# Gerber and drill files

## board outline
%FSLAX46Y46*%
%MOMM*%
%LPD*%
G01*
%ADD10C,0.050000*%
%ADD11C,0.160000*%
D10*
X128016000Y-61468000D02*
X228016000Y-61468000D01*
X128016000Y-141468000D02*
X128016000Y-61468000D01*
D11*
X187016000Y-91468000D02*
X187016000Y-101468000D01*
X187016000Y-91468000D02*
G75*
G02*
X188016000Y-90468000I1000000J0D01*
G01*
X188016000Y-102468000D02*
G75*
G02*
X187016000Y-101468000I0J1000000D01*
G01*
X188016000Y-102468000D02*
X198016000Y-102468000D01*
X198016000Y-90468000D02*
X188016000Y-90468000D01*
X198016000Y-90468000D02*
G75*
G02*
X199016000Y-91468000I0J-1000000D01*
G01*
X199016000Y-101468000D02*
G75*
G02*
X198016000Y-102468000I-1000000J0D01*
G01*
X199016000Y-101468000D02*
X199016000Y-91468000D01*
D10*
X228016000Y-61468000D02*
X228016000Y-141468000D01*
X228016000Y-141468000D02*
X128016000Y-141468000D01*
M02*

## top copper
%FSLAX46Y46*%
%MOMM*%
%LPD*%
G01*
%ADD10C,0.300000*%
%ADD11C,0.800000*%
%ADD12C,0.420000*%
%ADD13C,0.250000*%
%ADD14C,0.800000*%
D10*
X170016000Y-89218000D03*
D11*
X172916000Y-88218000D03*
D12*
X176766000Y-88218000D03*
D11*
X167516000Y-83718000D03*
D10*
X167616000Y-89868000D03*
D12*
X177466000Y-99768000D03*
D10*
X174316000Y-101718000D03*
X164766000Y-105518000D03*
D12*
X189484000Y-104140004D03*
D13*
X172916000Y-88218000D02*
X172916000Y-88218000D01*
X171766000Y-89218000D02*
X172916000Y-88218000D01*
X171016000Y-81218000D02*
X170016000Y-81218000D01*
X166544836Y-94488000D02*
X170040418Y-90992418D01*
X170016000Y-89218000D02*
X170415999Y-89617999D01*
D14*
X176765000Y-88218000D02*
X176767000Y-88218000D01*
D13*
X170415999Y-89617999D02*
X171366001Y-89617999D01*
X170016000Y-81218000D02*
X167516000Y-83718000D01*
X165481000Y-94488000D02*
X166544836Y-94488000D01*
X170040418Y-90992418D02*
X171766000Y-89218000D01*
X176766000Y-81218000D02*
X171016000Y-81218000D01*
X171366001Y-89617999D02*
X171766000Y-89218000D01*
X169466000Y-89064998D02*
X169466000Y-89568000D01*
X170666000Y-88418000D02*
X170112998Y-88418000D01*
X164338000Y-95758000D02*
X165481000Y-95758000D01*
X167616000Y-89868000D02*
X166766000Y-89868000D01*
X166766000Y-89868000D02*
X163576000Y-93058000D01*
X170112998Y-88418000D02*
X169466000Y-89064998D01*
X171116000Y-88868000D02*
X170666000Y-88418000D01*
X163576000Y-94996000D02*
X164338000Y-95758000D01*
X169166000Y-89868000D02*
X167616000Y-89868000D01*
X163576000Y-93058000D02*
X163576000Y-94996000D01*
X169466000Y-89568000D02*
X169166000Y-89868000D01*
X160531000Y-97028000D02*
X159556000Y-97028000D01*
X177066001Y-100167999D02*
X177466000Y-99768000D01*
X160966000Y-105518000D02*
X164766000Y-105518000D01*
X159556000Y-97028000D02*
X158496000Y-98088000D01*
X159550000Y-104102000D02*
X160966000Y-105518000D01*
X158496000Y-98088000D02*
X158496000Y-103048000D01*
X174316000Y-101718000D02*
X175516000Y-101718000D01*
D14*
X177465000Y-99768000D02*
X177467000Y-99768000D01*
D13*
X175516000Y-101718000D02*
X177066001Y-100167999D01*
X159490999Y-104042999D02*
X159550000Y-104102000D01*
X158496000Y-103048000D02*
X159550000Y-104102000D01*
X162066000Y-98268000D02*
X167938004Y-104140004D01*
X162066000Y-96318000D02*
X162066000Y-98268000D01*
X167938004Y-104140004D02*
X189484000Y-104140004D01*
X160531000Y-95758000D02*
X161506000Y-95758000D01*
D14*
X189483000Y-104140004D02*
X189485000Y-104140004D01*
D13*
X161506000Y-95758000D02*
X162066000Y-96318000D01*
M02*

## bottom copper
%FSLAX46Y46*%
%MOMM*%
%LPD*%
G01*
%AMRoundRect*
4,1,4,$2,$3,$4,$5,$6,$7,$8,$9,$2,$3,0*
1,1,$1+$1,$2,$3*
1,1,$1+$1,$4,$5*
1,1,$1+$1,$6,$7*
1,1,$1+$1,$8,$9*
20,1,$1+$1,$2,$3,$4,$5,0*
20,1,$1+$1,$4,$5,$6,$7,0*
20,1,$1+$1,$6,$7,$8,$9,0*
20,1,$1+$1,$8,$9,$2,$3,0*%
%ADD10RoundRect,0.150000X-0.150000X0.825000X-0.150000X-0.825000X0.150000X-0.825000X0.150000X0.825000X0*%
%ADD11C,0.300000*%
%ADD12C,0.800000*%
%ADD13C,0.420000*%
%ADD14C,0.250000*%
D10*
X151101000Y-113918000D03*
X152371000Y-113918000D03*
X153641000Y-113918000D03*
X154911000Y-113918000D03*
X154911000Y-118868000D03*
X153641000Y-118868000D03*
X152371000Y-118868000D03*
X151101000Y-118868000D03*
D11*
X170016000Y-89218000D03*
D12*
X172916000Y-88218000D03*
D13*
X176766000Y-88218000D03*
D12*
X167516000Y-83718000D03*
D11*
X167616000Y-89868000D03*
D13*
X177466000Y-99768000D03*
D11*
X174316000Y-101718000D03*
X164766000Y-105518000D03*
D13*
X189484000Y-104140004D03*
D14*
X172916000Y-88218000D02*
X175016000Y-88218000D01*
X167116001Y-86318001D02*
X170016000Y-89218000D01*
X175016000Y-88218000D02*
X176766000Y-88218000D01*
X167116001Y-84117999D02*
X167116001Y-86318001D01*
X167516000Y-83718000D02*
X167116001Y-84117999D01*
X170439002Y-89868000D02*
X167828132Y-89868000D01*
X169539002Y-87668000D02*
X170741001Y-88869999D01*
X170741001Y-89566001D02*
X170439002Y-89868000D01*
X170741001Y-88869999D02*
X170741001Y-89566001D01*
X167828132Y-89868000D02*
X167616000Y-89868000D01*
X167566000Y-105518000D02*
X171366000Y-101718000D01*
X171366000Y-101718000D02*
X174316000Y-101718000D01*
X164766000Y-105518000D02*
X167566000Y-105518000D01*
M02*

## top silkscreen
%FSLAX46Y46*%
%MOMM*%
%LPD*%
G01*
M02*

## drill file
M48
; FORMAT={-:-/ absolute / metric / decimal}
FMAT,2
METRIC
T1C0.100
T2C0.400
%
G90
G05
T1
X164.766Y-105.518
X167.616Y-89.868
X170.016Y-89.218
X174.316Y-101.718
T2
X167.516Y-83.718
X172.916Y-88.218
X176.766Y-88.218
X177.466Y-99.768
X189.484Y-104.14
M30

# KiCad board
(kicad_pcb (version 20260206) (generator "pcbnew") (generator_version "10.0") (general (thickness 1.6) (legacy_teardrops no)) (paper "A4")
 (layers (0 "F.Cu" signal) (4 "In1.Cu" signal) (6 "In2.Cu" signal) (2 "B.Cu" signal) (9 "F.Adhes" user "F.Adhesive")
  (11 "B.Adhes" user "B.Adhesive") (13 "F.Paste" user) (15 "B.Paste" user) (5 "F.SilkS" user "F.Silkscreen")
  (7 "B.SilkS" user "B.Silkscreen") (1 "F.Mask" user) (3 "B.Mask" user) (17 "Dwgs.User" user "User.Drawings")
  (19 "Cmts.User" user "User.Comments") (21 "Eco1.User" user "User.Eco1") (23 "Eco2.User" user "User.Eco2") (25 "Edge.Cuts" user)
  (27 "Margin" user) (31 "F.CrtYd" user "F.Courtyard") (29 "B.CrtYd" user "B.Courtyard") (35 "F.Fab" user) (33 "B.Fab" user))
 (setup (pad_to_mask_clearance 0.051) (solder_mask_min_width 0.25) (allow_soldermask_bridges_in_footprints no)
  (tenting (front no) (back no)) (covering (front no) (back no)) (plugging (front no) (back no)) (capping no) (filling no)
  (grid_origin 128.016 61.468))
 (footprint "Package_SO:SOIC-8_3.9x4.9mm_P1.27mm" (layer "B.Cu") (at 153.006 116.393 -90)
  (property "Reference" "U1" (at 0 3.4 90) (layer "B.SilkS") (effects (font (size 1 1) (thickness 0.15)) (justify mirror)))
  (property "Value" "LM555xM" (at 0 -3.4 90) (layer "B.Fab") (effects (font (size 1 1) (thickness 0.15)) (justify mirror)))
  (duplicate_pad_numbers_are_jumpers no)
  (pad "1" smd roundrect (at -2.475 1.905 270) (size 1.95 0.6) (layers "B.Cu" "B.Mask" "B.Paste") (roundrect_rratio 0.25)
   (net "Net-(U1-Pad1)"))
  (pad "2" smd roundrect (at -2.475 0.635 270) (size 1.95 0.6) (layers "B.Cu" "B.Mask" "B.Paste") (roundrect_rratio 0.25)
   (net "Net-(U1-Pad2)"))
  (pad "3" smd roundrect (at -2.475 -0.635 270) (size 1.95 0.6) (layers "B.Cu" "B.Mask" "B.Paste") (roundrect_rratio 0.25)
   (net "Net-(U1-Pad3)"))
  (pad "4" smd roundrect (at -2.475 -1.905 270) (size 1.95 0.6) (layers "B.Cu" "B.Mask" "B.Paste") (roundrect_rratio 0.25)
   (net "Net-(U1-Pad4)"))
  (pad "5" smd roundrect (at 2.475 -1.905 270) (size 1.95 0.6) (layers "B.Cu" "B.Mask" "B.Paste") (roundrect_rratio 0.25)
   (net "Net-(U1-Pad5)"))
  (pad "6" smd roundrect (at 2.475 -0.635 270) (size 1.95 0.6) (layers "B.Cu" "B.Mask" "B.Paste") (roundrect_rratio 0.25)
   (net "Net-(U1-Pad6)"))
  (pad "7" smd roundrect (at 2.475 0.635 270) (size 1.95 0.6) (layers "B.Cu" "B.Mask" "B.Paste") (roundrect_rratio 0.25)
   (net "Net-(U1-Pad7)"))
  (pad "8" smd roundrect (at 2.475 1.905 270) (size 1.95 0.6) (layers "B.Cu" "B.Mask" "B.Paste") (roundrect_rratio 0.25)
   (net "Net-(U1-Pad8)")))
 (gr_line (start 128.016 61.468) (end 228.016 61.468) (stroke (width 0.05) (type solid)) (layer "Edge.Cuts"))
 (gr_line (start 128.016 141.468) (end 128.016 61.468) (stroke (width 0.05) (type solid)) (layer "Edge.Cuts"))
 (gr_line (start 187.016 91.468) (end 187.016 101.468) (stroke (width 0.16) (type solid)) (layer "Edge.Cuts"))
 (gr_arc (start 187.016 91.468) (mid 187.308893 90.760893) (end 188.016 90.468) (stroke (width 0.16) (type solid)) (layer "Edge.Cuts"))
 (gr_arc (start 188.016 102.468) (mid 187.308893 102.175107) (end 187.016 101.468) (stroke (width 0.16) (type solid)) (layer "Edge.Cuts"))
 (gr_line (start 188.016 102.468) (end 198.016 102.468) (stroke (width 0.16) (type solid)) (layer "Edge.Cuts"))
 (gr_line (start 198.016 90.468) (end 188.016 90.468) (stroke (width 0.16) (type solid)) (layer "Edge.Cuts"))
 (gr_arc (start 198.016 90.468) (mid 198.723107 90.760893) (end 199.016 91.468) (stroke (width 0.16) (type solid)) (layer "Edge.Cuts"))
 (gr_arc (start 199.016 101.468) (mid 198.723107 102.175107) (end 198.016 102.468) (stroke (width 0.16) (type solid)) (layer "Edge.Cuts"))
 (gr_line (start 199.016 101.468) (end 199.016 91.468) (stroke (width 0.16) (type solid)) (layer "Edge.Cuts"))
 (gr_line (start 228.016 61.468) (end 228.016 141.468) (stroke (width 0.05) (type solid)) (layer "Edge.Cuts"))
 (gr_line (start 228.016 141.468) (end 128.016 141.468) (stroke (width 0.05) (type solid)) (layer "Edge.Cuts"))
 (segment (start 172.916 88.218) (end 172.916 88.218) (width 0.25) (layer "F.Cu") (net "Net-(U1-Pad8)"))
 (segment (start 171.766 89.218) (end 172.916 88.218) (width 0.25) (layer "F.Cu") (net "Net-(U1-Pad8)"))
 (segment (start 171.016 81.218) (end 170.016 81.218) (width 0.25) (layer "F.Cu") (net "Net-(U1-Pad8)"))
 (segment (start 166.544836 94.488) (end 170.040418 90.992418) (width 0.25) (layer "F.Cu") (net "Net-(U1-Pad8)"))
 (segment (start 170.016 89.218) (end 170.415999 89.617999) (width 0.25) (layer "F.Cu") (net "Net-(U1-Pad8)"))
 (segment (start 176.765 88.218) (end 176.767 88.218) (width 0.8) (layer "F.Cu") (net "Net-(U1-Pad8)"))
 (segment (start 170.415999 89.617999) (end 171.366001 89.617999) (width 0.25) (layer "F.Cu") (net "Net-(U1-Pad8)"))
 (segment (start 170.016 81.218) (end 167.516 83.718) (width 0.25) (layer "F.Cu") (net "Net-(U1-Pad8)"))
 (segment (start 165.481 94.488) (end 166.544836 94.488) (width 0.25) (layer "F.Cu") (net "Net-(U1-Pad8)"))
 (segment (start 170.040418 90.992418) (end 171.766 89.218) (width 0.25) (layer "F.Cu") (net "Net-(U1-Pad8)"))
 (segment (start 176.766 81.218) (end 171.016 81.218) (width 0.25) (layer "F.Cu") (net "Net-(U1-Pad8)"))
 (segment (start 171.366001 89.617999) (end 171.766 89.218) (width 0.25) (layer "F.Cu") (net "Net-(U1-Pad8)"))
 (via (at 170.016 89.218) (size 0.3) (drill 0.1) (layers "F.Cu" "B.Cu") (capping no) (covering (front no) (back no))
  (plugging (front no) (back no)) (filling no) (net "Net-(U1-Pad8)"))
 (via (at 172.916 88.218) (size 0.8) (drill 0.4) (layers "F.Cu" "B.Cu") (capping no) (covering (front no) (back no))
  (plugging (front no) (back no)) (filling no) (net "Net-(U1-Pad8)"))
 (via (at 176.766 88.218) (size 0.42) (drill 0.4) (layers "F.Cu" "B.Cu") (capping no) (covering (front no) (back no))
  (plugging (front no) (back no)) (filling no) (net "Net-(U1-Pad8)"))
 (via (at 167.516 83.718) (size 0.8) (drill 0.4) (layers "F.Cu" "B.Cu") (capping no) (covering (front no) (back no))
  (plugging (front no) (back no)) (filling no) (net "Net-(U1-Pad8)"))
 (segment (start 172.916 88.218) (end 175.016 88.218) (width 0.25) (layer "B.Cu") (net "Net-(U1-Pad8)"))
 (segment (start 167.116001 86.318001) (end 170.016 89.218) (width 0.25) (layer "B.Cu") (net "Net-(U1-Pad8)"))
 (segment (start 175.016 88.218) (end 176.766 88.218) (width 0.25) (layer "B.Cu") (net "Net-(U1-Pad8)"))
 (segment (start 167.116001 84.117999) (end 167.116001 86.318001) (width 0.25) (layer "B.Cu") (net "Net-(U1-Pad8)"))
 (segment (start 167.516 83.718) (end 167.116001 84.117999) (width 0.25) (layer "B.Cu") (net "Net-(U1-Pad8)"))
 (segment (start 169.466 89.064998) (end 169.466 89.568) (width 0.25) (layer "F.Cu") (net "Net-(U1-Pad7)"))
 (segment (start 170.666 88.418) (end 170.112998 88.418) (width 0.25) (layer "F.Cu") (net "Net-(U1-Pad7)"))
 (segment (start 164.338 95.758) (end 165.481 95.758) (width 0.25) (layer "F.Cu") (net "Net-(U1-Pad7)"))
 (segment (start 167.616 89.868) (end 166.766 89.868) (width 0.25) (layer "F.Cu") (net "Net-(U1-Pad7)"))
 (segment (start 166.766 89.868) (end 163.576 93.058) (width 0.25) (layer "F.Cu") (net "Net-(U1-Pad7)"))
 (segment (start 170.112998 88.418) (end 169.466 89.064998) (width 0.25) (layer "F.Cu") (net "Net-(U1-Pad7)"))
 (segment (start 171.116 88.868) (end 170.666 88.418) (width 0.25) (layer "F.Cu") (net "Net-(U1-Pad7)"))
 (segment (start 163.576 94.996) (end 164.338 95.758) (width 0.25) (layer "F.Cu") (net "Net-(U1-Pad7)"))
 (segment (start 169.166 89.868) (end 167.616 89.868) (width 0.25) (layer "F.Cu") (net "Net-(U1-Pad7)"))
 (segment (start 163.576 93.058) (end 163.576 94.996) (width 0.25) (layer "F.Cu") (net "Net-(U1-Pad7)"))
 (segment (start 169.466 89.568) (end 169.166 89.868) (width 0.25) (layer "F.Cu") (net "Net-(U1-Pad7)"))
 (via (at 167.616 89.868) (size 0.3) (drill 0.1) (layers "F.Cu" "B.Cu") (capping no) (covering (front no) (back no))
  (plugging (front no) (back no)) (filling no) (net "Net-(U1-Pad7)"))
 (segment (start 170.439002 89.868) (end 167.828132 89.868) (width 0.25) (layer "B.Cu") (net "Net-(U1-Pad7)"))
 (segment (start 169.539002 87.668) (end 170.741001 88.869999) (width 0.25) (layer "B.Cu") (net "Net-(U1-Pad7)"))
 (segment (start 170.741001 89.566001) (end 170.439002 89.868) (width 0.25) (layer "B.Cu") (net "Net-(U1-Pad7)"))
 (segment (start 170.741001 88.869999) (end 170.741001 89.566001) (width 0.25) (layer "B.Cu") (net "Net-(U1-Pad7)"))
 (segment (start 167.828132 89.868) (end 167.616 89.868) (width 0.25) (layer "B.Cu") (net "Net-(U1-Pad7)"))
 (segment (start 160.531 97.028) (end 159.556 97.028) (width 0.25) (layer "F.Cu") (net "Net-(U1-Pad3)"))
 (segment (start 177.066001 100.167999) (end 177.466 99.768) (width 0.25) (layer "F.Cu") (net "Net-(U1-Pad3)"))
 (segment (start 160.966 105.518) (end 164.766 105.518) (width 0.25) (layer "F.Cu") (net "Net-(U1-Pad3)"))
 (segment (start 159.556 97.028) (end 158.496 98.088) (width 0.25) (layer "F.Cu") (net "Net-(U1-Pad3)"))
 (segment (start 159.55 104.102) (end 160.966 105.518) (width 0.25) (layer "F.Cu") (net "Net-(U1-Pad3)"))
 (segment (start 158.496 98.088) (end 158.496 103.048) (width 0.25) (layer "F.Cu") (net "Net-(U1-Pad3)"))
 (segment (start 174.316 101.718) (end 175.516 101.718) (width 0.25) (layer "F.Cu") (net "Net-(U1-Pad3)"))
 (segment (start 177.465 99.768) (end 177.467 99.768) (width 0.8) (layer "F.Cu") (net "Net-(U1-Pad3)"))
 (segment (start 175.516 101.718) (end 177.066001 100.167999) (width 0.25) (layer "F.Cu") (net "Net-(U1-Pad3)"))
 (segment (start 159.490999 104.042999) (end 159.55 104.102) (width 0.25) (layer "F.Cu") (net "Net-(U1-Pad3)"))
 (segment (start 158.496 103.048) (end 159.55 104.102) (width 0.25) (layer "F.Cu") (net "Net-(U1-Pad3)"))
 (via (at 177.466 99.768) (size 0.42) (drill 0.4) (layers "F.Cu" "B.Cu") (capping no) (covering (front no) (back no))
  (plugging (front no) (back no)) (filling no) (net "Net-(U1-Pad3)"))
 (via (at 174.316 101.718) (size 0.3) (drill 0.1) (layers "F.Cu" "B.Cu") (capping no) (covering (front no) (back no))
  (plugging (front no) (back no)) (filling no) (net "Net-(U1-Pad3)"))
 (via (at 164.766 105.518) (size 0.3) (drill 0.1) (layers "F.Cu" "B.Cu") (capping no) (covering (front no) (back no))
  (plugging (front no) (back no)) (filling no) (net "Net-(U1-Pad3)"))
 (segment (start 167.566 105.518) (end 171.366 101.718) (width 0.25) (layer "B.Cu") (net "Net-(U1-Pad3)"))
 (segment (start 171.366 101.718) (end 174.316 101.718) (width 0.25) (layer "B.Cu") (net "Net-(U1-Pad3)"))
 (segment (start 164.766 105.518) (end 167.566 105.518) (width 0.25) (layer "B.Cu") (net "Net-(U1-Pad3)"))
 (segment (start 162.066 98.268) (end 167.938004 104.140004) (width 0.25) (layer "F.Cu") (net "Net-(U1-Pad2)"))
 (segment (start 162.066 96.318) (end 162.066 98.268) (width 0.25) (layer "F.Cu") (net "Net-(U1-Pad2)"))
 (segment (start 167.938004 104.140004) (end 189.484 104.140004) (width 0.25) (layer "F.Cu") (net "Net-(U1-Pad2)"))
 (segment (start 160.531 95.758) (end 161.506 95.758) (width 0.25) (layer "F.Cu") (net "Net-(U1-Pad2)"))
 (segment (start 189.483 104.140004) (end 189.485 104.140004) (width 0.8) (layer "F.Cu") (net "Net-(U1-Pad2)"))
 (segment (start 161.506 95.758) (end 162.066 96.318) (width 0.25) (layer "F.Cu") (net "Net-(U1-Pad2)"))
 (via (at 189.484 104.140004) (size 0.42) (drill 0.4) (layers "F.Cu" "B.Cu") (capping no) (covering (front no) (back no))
  (plugging (front no) (back no)) (filling no) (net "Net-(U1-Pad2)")))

